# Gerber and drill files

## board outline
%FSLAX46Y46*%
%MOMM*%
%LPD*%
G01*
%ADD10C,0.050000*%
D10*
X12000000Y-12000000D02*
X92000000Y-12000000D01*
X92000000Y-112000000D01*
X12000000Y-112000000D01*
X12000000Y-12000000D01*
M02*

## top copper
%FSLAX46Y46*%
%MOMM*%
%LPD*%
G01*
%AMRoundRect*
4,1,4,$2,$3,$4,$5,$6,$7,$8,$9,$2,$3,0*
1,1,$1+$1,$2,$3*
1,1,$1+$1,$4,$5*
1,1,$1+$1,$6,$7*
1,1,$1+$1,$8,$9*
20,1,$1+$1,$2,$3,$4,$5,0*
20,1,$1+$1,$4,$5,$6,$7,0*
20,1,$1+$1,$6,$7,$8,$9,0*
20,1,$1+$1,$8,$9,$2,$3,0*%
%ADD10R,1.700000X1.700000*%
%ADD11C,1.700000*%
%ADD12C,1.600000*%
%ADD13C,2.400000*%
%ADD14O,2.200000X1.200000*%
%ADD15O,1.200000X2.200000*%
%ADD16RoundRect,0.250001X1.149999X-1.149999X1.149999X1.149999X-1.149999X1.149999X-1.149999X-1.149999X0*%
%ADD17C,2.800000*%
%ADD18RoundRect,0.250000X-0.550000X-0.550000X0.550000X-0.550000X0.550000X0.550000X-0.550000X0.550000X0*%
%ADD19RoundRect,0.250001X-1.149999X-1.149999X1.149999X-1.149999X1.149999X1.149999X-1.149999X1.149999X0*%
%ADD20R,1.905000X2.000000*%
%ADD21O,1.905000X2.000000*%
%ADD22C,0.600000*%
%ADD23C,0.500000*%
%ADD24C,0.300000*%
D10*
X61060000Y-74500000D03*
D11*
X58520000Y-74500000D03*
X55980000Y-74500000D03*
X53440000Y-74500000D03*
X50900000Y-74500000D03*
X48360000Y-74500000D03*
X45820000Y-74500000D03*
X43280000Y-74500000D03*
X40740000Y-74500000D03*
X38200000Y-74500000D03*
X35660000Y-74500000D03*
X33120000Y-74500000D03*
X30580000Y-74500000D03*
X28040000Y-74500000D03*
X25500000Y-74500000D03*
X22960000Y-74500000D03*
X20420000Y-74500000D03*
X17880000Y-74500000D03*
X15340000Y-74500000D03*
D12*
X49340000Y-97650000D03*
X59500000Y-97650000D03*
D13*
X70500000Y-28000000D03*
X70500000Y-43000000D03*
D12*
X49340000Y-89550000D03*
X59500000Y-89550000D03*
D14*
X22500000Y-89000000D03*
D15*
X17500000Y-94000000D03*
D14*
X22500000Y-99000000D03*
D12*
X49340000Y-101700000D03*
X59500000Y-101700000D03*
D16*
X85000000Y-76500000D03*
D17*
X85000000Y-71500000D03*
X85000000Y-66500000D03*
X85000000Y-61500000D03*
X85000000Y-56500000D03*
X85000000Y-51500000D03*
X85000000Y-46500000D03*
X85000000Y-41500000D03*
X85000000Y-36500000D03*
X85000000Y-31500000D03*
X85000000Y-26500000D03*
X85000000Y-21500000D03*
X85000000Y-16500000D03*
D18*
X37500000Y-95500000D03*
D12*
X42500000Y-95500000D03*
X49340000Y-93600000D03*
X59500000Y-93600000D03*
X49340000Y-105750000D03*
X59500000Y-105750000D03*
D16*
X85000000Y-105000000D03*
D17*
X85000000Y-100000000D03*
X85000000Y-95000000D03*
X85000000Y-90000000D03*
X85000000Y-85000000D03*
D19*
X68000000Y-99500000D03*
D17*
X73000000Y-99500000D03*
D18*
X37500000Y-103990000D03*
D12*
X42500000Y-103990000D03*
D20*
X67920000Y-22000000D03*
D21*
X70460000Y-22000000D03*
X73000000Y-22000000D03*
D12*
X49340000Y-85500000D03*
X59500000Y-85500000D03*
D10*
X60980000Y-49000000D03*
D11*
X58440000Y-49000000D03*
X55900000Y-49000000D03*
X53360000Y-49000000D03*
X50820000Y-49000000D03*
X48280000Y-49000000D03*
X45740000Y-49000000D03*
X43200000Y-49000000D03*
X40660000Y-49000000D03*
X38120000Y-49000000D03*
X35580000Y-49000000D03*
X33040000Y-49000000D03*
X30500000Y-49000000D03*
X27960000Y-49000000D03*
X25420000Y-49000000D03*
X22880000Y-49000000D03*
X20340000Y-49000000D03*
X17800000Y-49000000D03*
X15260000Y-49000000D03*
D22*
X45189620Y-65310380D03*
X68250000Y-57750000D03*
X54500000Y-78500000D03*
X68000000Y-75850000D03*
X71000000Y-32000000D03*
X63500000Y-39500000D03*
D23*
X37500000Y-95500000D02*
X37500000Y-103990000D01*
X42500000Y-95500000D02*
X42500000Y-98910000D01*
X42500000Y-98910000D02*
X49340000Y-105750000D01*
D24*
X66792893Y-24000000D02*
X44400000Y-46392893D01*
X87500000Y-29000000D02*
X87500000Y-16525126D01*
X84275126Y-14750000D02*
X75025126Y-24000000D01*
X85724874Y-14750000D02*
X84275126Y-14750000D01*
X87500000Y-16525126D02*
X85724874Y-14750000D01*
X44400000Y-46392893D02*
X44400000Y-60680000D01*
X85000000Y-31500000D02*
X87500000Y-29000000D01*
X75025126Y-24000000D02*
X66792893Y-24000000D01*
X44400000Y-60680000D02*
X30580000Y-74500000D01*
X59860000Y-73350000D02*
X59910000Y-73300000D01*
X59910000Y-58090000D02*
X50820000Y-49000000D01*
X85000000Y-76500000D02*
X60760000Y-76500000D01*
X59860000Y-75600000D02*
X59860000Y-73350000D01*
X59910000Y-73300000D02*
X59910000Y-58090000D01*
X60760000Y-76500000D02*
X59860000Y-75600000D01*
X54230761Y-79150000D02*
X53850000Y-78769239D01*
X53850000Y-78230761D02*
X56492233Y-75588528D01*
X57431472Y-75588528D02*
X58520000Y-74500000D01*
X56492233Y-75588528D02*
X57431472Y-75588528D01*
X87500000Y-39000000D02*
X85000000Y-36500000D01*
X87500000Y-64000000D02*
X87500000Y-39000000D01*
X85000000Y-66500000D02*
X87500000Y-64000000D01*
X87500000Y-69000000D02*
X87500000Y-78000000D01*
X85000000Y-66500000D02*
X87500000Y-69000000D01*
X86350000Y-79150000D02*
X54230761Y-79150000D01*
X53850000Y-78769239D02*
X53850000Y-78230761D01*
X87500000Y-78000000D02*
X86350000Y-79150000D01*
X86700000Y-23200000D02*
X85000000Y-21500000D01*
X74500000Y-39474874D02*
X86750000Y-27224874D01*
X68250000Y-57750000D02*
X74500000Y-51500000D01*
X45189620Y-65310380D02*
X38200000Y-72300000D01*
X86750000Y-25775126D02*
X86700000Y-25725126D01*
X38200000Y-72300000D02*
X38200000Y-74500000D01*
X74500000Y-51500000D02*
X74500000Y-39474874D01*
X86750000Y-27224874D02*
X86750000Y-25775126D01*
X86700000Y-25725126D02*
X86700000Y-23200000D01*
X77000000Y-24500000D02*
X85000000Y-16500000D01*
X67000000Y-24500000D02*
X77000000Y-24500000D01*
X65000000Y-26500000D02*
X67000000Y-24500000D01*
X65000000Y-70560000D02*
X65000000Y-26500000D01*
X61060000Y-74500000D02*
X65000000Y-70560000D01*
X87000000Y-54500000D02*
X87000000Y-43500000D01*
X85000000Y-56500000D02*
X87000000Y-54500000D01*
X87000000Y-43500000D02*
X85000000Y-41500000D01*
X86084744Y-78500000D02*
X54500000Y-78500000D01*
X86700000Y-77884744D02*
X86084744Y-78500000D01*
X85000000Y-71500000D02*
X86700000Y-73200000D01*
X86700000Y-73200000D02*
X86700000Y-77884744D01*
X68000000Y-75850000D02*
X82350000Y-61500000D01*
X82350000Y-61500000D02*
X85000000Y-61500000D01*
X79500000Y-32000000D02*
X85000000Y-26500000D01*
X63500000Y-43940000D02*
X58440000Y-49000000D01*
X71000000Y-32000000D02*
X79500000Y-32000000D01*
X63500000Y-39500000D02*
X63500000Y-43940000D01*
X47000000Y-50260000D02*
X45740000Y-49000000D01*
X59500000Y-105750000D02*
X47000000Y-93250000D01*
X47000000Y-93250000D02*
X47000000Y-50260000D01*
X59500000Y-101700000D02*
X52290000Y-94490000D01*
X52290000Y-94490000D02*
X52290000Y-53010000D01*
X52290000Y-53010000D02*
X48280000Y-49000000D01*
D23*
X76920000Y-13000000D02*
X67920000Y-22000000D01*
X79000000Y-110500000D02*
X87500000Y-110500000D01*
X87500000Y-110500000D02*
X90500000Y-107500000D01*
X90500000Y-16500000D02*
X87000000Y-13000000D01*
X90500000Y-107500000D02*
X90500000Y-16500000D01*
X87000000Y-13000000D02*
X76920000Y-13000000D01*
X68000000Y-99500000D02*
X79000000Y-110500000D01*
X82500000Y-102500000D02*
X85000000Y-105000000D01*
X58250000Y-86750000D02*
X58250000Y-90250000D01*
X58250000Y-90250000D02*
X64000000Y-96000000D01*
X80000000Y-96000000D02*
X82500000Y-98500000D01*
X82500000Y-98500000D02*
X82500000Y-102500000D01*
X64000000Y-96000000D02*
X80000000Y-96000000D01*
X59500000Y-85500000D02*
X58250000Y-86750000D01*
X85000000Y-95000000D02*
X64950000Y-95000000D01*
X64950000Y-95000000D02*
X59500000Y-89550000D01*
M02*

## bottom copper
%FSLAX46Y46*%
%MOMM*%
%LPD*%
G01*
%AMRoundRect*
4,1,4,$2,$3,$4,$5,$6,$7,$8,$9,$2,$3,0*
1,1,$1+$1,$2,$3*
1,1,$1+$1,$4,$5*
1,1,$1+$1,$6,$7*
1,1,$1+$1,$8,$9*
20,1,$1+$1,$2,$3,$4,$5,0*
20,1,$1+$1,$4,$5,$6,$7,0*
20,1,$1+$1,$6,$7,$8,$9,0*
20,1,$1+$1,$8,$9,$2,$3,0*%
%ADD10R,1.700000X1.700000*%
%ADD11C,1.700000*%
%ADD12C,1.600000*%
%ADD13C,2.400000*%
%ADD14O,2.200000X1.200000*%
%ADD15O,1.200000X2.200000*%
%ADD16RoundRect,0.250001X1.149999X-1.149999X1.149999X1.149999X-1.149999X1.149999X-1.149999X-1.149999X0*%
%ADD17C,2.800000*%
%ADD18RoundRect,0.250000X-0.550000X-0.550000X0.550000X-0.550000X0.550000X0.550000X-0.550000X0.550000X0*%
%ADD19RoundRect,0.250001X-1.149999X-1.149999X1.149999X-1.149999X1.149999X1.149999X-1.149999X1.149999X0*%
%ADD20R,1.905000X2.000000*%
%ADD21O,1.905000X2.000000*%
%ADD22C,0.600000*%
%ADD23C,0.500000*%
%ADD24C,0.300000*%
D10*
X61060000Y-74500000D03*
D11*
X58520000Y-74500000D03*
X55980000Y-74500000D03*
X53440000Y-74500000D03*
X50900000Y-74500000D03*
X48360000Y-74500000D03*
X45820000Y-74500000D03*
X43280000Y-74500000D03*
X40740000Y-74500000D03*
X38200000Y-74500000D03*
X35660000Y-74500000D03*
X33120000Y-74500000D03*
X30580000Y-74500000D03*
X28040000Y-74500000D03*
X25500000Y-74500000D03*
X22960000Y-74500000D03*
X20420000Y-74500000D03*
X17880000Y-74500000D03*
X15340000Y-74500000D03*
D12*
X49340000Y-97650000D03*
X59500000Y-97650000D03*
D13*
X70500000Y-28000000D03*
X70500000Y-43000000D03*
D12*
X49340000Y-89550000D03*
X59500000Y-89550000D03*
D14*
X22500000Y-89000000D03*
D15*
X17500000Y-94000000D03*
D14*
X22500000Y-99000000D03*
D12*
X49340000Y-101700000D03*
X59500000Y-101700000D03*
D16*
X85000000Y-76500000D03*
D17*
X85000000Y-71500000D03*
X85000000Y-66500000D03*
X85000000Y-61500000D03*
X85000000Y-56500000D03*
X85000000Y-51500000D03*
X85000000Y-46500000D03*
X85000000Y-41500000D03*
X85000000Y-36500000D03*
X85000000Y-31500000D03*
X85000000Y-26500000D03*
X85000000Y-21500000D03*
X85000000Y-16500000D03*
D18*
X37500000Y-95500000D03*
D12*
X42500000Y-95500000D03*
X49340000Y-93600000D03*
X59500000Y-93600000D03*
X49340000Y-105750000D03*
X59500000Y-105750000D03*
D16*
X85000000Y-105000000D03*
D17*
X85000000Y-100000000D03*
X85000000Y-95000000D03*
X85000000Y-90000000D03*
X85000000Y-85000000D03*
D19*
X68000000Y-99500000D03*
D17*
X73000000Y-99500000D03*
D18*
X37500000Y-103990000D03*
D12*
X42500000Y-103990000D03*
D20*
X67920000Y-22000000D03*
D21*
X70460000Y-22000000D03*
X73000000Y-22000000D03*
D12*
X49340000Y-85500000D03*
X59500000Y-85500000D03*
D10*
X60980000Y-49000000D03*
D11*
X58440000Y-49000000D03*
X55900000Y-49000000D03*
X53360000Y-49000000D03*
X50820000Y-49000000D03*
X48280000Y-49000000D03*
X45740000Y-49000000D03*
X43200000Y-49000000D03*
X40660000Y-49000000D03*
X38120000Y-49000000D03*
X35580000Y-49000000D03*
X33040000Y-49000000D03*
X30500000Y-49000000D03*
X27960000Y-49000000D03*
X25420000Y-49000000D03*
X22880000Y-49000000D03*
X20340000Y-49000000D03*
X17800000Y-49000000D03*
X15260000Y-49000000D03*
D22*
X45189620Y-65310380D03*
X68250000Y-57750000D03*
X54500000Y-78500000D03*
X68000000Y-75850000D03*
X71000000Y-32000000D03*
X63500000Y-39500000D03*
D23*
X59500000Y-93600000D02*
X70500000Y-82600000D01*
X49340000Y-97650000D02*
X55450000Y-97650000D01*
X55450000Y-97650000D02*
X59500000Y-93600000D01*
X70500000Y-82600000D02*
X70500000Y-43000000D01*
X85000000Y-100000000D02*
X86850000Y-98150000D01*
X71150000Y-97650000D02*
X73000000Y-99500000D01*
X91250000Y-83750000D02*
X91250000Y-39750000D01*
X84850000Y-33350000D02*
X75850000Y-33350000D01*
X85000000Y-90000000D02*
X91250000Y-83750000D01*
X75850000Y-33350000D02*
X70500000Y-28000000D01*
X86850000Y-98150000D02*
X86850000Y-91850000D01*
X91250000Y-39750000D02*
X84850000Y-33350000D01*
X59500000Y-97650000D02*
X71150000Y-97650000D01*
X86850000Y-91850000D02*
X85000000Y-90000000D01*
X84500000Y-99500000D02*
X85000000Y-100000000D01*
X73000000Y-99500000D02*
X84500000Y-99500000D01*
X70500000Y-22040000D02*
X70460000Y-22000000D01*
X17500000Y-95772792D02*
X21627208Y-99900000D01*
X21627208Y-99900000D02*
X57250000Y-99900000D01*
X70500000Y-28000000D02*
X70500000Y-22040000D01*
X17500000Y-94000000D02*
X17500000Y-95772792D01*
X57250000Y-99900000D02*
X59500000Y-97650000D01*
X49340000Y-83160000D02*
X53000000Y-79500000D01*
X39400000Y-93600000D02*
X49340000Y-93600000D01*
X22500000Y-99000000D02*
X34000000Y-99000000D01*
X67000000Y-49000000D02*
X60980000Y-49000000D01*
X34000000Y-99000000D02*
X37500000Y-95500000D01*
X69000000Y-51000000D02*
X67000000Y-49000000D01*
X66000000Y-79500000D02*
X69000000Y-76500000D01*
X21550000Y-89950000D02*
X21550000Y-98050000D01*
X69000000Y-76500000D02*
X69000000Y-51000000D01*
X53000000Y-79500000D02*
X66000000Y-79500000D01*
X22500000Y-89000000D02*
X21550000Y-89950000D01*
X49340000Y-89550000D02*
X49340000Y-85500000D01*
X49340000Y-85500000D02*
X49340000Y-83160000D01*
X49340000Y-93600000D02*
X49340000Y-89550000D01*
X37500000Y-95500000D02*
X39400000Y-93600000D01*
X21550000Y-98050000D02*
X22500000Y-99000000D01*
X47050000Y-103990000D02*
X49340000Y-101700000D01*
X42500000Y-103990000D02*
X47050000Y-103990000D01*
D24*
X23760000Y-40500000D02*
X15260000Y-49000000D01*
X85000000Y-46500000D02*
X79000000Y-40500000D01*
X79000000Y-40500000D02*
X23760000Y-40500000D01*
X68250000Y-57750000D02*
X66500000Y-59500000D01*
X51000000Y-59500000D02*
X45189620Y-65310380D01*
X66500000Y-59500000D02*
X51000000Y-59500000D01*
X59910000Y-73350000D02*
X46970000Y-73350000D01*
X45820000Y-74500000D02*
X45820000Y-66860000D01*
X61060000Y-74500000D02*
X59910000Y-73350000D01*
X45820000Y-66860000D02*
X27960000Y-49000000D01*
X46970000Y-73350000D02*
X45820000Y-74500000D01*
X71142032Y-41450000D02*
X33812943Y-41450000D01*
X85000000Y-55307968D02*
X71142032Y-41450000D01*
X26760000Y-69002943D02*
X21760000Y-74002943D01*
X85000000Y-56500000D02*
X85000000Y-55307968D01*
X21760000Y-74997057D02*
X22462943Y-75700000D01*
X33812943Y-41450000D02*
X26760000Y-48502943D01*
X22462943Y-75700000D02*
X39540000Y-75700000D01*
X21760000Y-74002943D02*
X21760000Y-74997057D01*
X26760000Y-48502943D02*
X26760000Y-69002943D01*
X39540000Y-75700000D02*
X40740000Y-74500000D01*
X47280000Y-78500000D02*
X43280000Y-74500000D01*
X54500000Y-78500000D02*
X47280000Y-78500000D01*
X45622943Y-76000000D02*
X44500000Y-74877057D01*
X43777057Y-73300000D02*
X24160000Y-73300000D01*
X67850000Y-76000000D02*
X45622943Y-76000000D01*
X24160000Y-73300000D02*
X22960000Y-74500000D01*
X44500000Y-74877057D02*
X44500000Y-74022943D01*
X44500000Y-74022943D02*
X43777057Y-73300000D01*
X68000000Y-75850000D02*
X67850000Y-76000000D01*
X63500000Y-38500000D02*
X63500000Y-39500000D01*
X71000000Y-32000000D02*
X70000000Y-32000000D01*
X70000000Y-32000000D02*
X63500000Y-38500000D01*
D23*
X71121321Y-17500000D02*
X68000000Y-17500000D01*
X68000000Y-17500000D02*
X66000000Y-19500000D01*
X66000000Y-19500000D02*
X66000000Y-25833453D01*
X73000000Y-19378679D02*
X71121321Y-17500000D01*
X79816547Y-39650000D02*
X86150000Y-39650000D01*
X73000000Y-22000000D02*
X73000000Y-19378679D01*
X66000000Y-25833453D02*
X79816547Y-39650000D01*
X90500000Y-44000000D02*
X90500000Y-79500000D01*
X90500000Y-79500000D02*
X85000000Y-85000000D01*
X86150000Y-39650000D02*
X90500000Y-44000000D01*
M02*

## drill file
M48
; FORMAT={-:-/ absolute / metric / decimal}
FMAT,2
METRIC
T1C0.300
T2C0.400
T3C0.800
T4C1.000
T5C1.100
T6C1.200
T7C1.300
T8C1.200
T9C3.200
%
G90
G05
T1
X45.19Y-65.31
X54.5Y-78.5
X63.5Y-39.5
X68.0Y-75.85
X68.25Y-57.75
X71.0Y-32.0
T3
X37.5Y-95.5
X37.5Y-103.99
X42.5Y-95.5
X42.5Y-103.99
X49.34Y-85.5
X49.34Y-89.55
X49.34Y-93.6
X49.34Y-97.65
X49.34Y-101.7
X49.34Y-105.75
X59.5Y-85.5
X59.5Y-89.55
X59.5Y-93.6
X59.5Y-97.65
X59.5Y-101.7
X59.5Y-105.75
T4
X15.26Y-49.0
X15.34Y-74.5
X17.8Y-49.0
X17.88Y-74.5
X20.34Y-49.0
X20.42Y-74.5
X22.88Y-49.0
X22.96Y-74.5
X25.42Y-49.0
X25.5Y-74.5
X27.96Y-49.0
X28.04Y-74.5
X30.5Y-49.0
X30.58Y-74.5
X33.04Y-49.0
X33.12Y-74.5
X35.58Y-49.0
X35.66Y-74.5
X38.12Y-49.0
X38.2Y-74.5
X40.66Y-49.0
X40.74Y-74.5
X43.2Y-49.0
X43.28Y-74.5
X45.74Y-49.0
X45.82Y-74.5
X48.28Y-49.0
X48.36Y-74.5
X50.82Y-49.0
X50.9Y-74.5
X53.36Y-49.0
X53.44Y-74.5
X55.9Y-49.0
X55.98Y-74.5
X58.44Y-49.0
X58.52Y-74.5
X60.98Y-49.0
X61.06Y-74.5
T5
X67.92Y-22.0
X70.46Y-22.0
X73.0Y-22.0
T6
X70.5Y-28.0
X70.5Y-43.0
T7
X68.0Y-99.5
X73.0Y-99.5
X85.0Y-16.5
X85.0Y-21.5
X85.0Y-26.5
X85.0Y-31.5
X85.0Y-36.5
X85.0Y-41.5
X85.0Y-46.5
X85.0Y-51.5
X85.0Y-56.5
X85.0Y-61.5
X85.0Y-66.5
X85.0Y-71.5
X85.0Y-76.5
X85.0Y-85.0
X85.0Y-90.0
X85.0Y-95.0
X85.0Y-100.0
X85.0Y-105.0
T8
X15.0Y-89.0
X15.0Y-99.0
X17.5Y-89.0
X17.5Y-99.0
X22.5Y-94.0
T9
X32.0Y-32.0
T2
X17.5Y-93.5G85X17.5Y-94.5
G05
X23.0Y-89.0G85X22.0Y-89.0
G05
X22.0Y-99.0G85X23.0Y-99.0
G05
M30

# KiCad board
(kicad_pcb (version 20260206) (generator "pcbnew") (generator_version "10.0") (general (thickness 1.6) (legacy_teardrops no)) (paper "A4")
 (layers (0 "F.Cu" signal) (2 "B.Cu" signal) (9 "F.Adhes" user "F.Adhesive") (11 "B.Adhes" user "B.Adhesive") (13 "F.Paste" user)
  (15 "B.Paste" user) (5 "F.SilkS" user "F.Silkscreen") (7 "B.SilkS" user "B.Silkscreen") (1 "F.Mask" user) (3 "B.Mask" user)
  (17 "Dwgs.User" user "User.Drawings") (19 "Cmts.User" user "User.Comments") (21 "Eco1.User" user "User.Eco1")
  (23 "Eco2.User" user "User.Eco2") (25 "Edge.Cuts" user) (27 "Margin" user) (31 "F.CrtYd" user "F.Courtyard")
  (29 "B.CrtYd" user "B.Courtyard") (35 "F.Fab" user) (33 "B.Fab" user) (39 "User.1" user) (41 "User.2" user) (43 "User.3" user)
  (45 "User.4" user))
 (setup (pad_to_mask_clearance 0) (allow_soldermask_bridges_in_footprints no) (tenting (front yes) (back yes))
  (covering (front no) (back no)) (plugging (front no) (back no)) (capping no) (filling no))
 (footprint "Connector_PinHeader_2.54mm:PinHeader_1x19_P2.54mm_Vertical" (layer "F.Cu") (at 61.06 74.5 -90)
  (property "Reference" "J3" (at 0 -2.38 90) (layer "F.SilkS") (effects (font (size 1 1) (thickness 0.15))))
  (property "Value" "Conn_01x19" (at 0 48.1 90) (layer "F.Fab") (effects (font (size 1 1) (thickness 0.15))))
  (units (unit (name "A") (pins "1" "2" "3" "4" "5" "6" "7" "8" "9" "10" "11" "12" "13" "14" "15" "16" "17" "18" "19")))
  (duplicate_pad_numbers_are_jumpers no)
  (pad "1" thru_hole rect (at 0 0 270) (size 1.7 1.7) (drill 1) (layers "*.Cu" "*.Mask") (remove_unused_layers no) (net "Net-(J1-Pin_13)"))
  (pad "2" thru_hole circle (at 0 2.54 270) (size 1.7 1.7) (drill 1) (layers "*.Cu" "*.Mask") (remove_unused_layers no)
   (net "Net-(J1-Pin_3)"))
  (pad "3" thru_hole circle (at 0 5.08 270) (size 1.7 1.7) (drill 1) (layers "*.Cu" "*.Mask") (remove_unused_layers no)
   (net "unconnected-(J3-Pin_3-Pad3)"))
  (pad "4" thru_hole circle (at 0 7.62 270) (size 1.7 1.7) (drill 1) (layers "*.Cu" "*.Mask") (remove_unused_layers no)
   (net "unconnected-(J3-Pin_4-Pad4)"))
  (pad "5" thru_hole circle (at 0 10.16 270) (size 1.7 1.7) (drill 1) (layers "*.Cu" "*.Mask") (remove_unused_layers no)
   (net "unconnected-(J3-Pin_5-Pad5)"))
  (pad "6" thru_hole circle (at 0 12.7 270) (size 1.7 1.7) (drill 1) (layers "*.Cu" "*.Mask") (remove_unused_layers no)
   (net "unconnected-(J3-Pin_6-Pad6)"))
  (pad "7" thru_hole circle (at 0 15.24 270) (size 1.7 1.7) (drill 1) (layers "*.Cu" "*.Mask") (remove_unused_layers no)
   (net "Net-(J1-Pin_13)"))
  (pad "8" thru_hole circle (at 0 17.78 270) (size 1.7 1.7) (drill 1) (layers "*.Cu" "*.Mask") (remove_unused_layers no)
   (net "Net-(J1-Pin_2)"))
  (pad "9" thru_hole circle (at 0 20.32 270) (size 1.7 1.7) (drill 1) (layers "*.Cu" "*.Mask") (remove_unused_layers no)
   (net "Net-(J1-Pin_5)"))
  (pad "10" thru_hole circle (at 0 22.86 270) (size 1.7 1.7) (drill 1) (layers "*.Cu" "*.Mask") (remove_unused_layers no)
   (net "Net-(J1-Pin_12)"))
  (pad "11" thru_hole circle (at 0 25.4 270) (size 1.7 1.7) (drill 1) (layers "*.Cu" "*.Mask") (remove_unused_layers no)
   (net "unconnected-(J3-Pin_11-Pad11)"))
  (pad "12" thru_hole circle (at 0 27.94 270) (size 1.7 1.7) (drill 1) (layers "*.Cu" "*.Mask") (remove_unused_layers no)
   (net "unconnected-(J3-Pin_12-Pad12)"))
  (pad "13" thru_hole circle (at 0 30.48 270) (size 1.7 1.7) (drill 1) (layers "*.Cu" "*.Mask") (remove_unused_layers no)
   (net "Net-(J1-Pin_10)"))
  (pad "14" thru_hole circle (at 0 33.02 270) (size 1.7 1.7) (drill 1) (layers "*.Cu" "*.Mask") (remove_unused_layers no)
   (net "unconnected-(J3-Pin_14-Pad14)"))
  (pad "15" thru_hole circle (at 0 35.56 270) (size 1.7 1.7) (drill 1) (layers "*.Cu" "*.Mask") (remove_unused_layers no)
   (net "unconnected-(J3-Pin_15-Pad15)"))
  (pad "16" thru_hole circle (at 0 38.1 270) (size 1.7 1.7) (drill 1) (layers "*.Cu" "*.Mask") (remove_unused_layers no)
   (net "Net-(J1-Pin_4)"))
  (pad "17" thru_hole circle (at 0 40.64 270) (size 1.7 1.7) (drill 1) (layers "*.Cu" "*.Mask") (remove_unused_layers no)
   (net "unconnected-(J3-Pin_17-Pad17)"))
  (pad "18" thru_hole circle (at 0 43.18 270) (size 1.7 1.7) (drill 1) (layers "*.Cu" "*.Mask") (remove_unused_layers no)
   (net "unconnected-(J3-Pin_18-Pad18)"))
  (pad "19" thru_hole circle (at 0 45.72 270) (size 1.7 1.7) (drill 1) (layers "*.Cu" "*.Mask") (remove_unused_layers no)
   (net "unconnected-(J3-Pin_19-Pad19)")))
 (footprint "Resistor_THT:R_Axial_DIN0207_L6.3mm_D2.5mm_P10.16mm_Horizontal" (layer "F.Cu") (at 49.34 97.65)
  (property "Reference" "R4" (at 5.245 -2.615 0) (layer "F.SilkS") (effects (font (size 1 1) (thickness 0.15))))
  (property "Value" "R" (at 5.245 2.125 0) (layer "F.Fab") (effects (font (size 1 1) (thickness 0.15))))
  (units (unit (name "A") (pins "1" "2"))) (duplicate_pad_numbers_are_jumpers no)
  (pad "1" thru_hole circle (at 0 0) (size 1.6 1.6) (drill 0.8) (layers "*.Cu" "*.Mask") (remove_unused_layers no) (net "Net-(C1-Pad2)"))
  (pad "2" thru_hole circle (at 10.16 0) (size 1.6 1.6) (drill 0.8) (layers "*.Cu" "*.Mask") (remove_unused_layers no) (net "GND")))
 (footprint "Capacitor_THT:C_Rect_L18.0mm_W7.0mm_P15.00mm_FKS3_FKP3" (layer "F.Cu") (at 70.5 28 -90)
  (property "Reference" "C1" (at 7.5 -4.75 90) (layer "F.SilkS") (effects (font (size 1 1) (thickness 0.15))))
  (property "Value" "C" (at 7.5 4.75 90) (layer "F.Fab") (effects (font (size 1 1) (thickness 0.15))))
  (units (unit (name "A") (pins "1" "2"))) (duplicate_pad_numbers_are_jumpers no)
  (pad "1" thru_hole circle (at 0 0 270) (size 2.4 2.4) (drill 1.2) (layers "*.Cu" "*.Mask") (remove_unused_layers no) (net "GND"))
  (pad "2" thru_hole circle (at 15 0 270) (size 2.4 2.4) (drill 1.2) (layers "*.Cu" "*.Mask") (remove_unused_layers no)
   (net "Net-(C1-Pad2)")))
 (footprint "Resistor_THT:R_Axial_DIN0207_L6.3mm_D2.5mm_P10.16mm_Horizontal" (layer "F.Cu") (at 49.34 89.55)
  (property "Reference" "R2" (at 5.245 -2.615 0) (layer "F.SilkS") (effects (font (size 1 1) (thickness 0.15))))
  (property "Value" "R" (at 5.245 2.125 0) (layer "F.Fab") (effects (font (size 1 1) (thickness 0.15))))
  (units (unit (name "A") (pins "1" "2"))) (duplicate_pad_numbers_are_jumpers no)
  (pad "1" thru_hole circle (at 0 0) (size 1.6 1.6) (drill 0.8) (layers "*.Cu" "*.Mask") (remove_unused_layers no) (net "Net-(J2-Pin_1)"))
  (pad "2" thru_hole circle (at 10.16 0) (size 1.6 1.6) (drill 0.8) (layers "*.Cu" "*.Mask") (remove_unused_layers no) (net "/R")))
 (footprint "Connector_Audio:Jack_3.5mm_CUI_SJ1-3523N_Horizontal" (layer "F.Cu") (at 17.5 94 -90)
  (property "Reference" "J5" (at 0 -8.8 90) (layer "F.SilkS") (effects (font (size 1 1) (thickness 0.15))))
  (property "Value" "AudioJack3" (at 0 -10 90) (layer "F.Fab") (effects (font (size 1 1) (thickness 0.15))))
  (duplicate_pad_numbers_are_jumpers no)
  (pad "" np_thru_hole circle (at -5 0 270) (size 1.2 1.2) (drill 1.2) (layers "*.Cu" "*.Mask"))
  (pad "" np_thru_hole circle (at -5 2.5 270) (size 1.2 1.2) (drill 1.2) (layers "*.Cu" "*.Mask"))
  (pad "" np_thru_hole circle (at 0 -5 270) (size 1.2 1.2) (drill 1.2) (layers "*.Cu" "*.Mask"))
  (pad "" np_thru_hole circle (at 5 0 270) (size 1.2 1.2) (drill 1.2) (layers "*.Cu" "*.Mask"))
  (pad "" np_thru_hole circle (at 5 2.5 270) (size 1.2 1.2) (drill 1.2) (layers "*.Cu" "*.Mask"))
  (pad "R" thru_hole oval (at -5 -5 270) (size 1.2 2.2) (drill oval 0.4 1.4) (layers "*.Cu" "*.Mask") (remove_unused_layers no)
   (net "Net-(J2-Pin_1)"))
  (pad "S" thru_hole oval (at 0 0 270) (size 2.2 1.2) (drill oval 1.4 0.4) (layers "*.Cu" "*.Mask") (remove_unused_layers no) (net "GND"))
  (pad "T" thru_hole oval (at 5 -5 90) (size 1.2 2.2) (drill oval 0.4 1.4) (layers "*.Cu" "*.Mask") (remove_unused_layers no)
   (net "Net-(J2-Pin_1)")))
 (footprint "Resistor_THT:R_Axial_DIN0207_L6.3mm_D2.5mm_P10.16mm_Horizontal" (layer "F.Cu") (at 49.34 101.7)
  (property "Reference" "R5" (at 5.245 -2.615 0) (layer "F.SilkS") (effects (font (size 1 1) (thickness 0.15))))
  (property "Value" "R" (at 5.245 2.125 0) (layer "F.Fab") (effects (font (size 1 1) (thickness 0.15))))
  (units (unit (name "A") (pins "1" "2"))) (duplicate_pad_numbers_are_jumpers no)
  (pad "1" thru_hole circle (at 0 0) (size 1.6 1.6) (drill 0.8) (layers "*.Cu" "*.Mask") (remove_unused_layers no) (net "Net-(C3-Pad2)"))
  (pad "2" thru_hole circle (at 10.16 0) (size 1.6 1.6) (drill 0.8) (layers "*.Cu" "*.Mask") (remove_unused_layers no)
   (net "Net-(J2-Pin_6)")))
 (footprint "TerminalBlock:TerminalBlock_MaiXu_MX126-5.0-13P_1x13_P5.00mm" (layer "F.Cu") (at 85 76.5 90)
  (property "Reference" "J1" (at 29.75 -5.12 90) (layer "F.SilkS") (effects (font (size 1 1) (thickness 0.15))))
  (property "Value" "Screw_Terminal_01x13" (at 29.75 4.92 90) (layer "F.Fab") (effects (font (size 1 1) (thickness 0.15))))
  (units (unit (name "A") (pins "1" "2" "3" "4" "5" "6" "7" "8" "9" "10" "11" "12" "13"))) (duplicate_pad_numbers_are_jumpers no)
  (pad "1" thru_hole roundrect (at 0 0 90) (size 2.8 2.8) (drill 1.3) (layers "*.Cu" "*.Mask") (remove_unused_layers no)
   (roundrect_rratio 0.089286) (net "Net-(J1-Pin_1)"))
  (pad "2" thru_hole circle (at 5 0 90) (size 2.8 2.8) (drill 1.3) (layers "*.Cu" "*.Mask") (remove_unused_layers no) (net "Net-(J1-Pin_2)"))
  (pad "3" thru_hole circle (at 10 0 90) (size 2.8 2.8) (drill 1.3) (layers "*.Cu" "*.Mask") (remove_unused_layers no)
   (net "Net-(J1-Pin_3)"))
  (pad "4" thru_hole circle (at 15 0 90) (size 2.8 2.8) (drill 1.3) (layers "*.Cu" "*.Mask") (remove_unused_layers no)
   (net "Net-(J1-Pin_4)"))
  (pad "5" thru_hole circle (at 20 0 90) (size 2.8 2.8) (drill 1.3) (layers "*.Cu" "*.Mask") (remove_unused_layers no)
   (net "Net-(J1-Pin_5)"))
  (pad "6" thru_hole circle (at 25 0 90) (size 2.8 2.8) (drill 1.3) (layers "*.Cu" "*.Mask") (remove_unused_layers no)
   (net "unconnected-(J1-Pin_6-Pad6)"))
  (pad "7" thru_hole circle (at 30 0 90) (size 2.8 2.8) (drill 1.3) (layers "*.Cu" "*.Mask") (remove_unused_layers no)
   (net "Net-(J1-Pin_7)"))
  (pad "8" thru_hole circle (at 35 0 90) (size 2.8 2.8) (drill 1.3) (layers "*.Cu" "*.Mask") (remove_unused_layers no)
   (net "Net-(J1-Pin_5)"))
  (pad "9" thru_hole circle (at 40 0 90) (size 2.8 2.8) (drill 1.3) (layers "*.Cu" "*.Mask") (remove_unused_layers no)
   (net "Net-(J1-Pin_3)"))
  (pad "10" thru_hole circle (at 45 0 90) (size 2.8 2.8) (drill 1.3) (layers "*.Cu" "*.Mask") (remove_unused_layers no)
   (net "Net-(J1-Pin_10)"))
  (pad "11" thru_hole circle (at 50 0 90) (size 2.8 2.8) (drill 1.3) (layers "*.Cu" "*.Mask") (remove_unused_layers no)
   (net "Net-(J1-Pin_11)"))
  (pad "12" thru_hole circle (at 55 0 90) (size 2.8 2.8) (drill 1.3) (layers "*.Cu" "*.Mask") (remove_unused_layers no)
   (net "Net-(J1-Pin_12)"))
  (pad "13" thru_hole circle (at 60 0 90) (size 2.8 2.8) (drill 1.3) (layers "*.Cu" "*.Mask") (remove_unused_layers no)
   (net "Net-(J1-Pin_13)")))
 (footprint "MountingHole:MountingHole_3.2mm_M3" (layer "F.Cu") (at 32 32)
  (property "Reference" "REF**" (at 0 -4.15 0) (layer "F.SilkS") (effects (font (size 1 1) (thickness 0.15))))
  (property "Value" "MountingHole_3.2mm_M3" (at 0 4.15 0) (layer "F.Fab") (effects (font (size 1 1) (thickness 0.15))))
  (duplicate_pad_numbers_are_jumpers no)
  (pad "" np_thru_hole circle (at 0 0) (size 3.2 3.2) (drill 3.2) (layers "*.Cu" "*.Mask")))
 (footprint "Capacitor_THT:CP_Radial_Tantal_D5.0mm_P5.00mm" (layer "F.Cu") (at 37.5 95.5)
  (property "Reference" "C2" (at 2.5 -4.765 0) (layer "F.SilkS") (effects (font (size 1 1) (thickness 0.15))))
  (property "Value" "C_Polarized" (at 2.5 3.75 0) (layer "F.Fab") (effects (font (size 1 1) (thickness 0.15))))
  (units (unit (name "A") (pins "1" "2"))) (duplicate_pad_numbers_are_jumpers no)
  (pad "1" thru_hole roundrect (at 0 0) (size 1.6 1.6) (drill 0.8) (layers "*.Cu" "*.Mask") (remove_unused_layers no)
   (roundrect_rratio 0.15625) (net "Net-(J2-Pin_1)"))
  (pad "2" thru_hole circle (at 5 0) (size 1.6 1.6) (drill 0.8) (layers "*.Cu" "*.Mask") (remove_unused_layers no) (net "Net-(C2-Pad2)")))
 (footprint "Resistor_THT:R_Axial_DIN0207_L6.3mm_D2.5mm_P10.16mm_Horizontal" (layer "F.Cu") (at 49.34 93.6)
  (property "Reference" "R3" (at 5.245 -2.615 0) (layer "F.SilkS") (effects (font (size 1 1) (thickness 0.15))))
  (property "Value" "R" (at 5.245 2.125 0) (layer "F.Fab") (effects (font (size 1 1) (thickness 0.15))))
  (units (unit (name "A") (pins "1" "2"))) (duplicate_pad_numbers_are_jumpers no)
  (pad "1" thru_hole circle (at 0 0) (size 1.6 1.6) (drill 0.8) (layers "*.Cu" "*.Mask") (remove_unused_layers no) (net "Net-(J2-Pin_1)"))
  (pad "2" thru_hole circle (at 10.16 0) (size 1.6 1.6) (drill 0.8) (layers "*.Cu" "*.Mask") (remove_unused_layers no) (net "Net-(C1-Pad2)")))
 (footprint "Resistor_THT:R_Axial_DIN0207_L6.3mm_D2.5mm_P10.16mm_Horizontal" (layer "F.Cu") (at 49.34 105.75)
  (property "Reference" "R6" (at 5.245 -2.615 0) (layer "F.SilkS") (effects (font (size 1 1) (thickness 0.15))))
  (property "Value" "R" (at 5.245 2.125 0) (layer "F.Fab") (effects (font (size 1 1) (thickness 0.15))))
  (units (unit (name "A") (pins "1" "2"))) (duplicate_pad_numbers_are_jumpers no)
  (pad "1" thru_hole circle (at 0 0) (size 1.6 1.6) (drill 0.8) (layers "*.Cu" "*.Mask") (remove_unused_layers no) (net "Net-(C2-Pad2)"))
  (pad "2" thru_hole circle (at 10.16 0) (size 1.6 1.6) (drill 0.8) (layers "*.Cu" "*.Mask") (remove_unused_layers no)
   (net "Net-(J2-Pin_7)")))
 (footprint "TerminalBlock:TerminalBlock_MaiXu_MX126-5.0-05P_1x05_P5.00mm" (layer "F.Cu") (at 85 105 90)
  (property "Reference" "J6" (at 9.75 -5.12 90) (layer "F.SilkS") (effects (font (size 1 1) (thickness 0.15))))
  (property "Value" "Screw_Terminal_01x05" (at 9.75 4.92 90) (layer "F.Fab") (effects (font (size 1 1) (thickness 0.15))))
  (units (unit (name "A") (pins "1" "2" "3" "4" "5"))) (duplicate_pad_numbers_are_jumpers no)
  (pad "1" thru_hole roundrect (at 0 0 90) (size 2.8 2.8) (drill 1.3) (layers "*.Cu" "*.Mask") (remove_unused_layers no)
   (roundrect_rratio 0.089286) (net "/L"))
  (pad "2" thru_hole circle (at 5 0 90) (size 2.8 2.8) (drill 1.3) (layers "*.Cu" "*.Mask") (remove_unused_layers no) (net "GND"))
  (pad "3" thru_hole circle (at 10 0 90) (size 2.8 2.8) (drill 1.3) (layers "*.Cu" "*.Mask") (remove_unused_layers no) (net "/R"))
  (pad "4" thru_hole circle (at 15 0 90) (size 2.8 2.8) (drill 1.3) (layers "*.Cu" "*.Mask") (remove_unused_layers no) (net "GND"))
  (pad "5" thru_hole circle (at 20 0 90) (size 2.8 2.8) (drill 1.3) (layers "*.Cu" "*.Mask") (remove_unused_layers no) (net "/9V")))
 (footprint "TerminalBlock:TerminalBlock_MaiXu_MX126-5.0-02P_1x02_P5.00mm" (layer "F.Cu") (at 68 99.5)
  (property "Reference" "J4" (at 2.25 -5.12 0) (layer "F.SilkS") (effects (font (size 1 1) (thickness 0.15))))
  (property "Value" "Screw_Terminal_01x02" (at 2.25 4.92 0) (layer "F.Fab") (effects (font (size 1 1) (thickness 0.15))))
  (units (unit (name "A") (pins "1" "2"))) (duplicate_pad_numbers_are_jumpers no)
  (pad "1" thru_hole roundrect (at 0 0) (size 2.8 2.8) (drill 1.3) (layers "*.Cu" "*.Mask") (remove_unused_layers no)
   (roundrect_rratio 0.089286) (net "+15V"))
  (pad "2" thru_hole circle (at 5 0) (size 2.8 2.8) (drill 1.3) (layers "*.Cu" "*.Mask") (remove_unused_layers no) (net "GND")))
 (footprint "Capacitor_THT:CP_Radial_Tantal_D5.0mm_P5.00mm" (layer "F.Cu") (at 37.5 103.99)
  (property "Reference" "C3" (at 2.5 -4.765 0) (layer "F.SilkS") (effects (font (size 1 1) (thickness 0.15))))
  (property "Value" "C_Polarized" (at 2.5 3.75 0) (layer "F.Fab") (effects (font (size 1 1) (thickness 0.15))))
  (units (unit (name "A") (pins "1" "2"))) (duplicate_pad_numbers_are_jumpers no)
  (pad "1" thru_hole roundrect (at 0 0) (size 1.6 1.6) (drill 0.8) (layers "*.Cu" "*.Mask") (remove_unused_layers no)
   (roundrect_rratio 0.15625) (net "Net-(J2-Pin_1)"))
  (pad "2" thru_hole circle (at 5 0) (size 1.6 1.6) (drill 0.8) (layers "*.Cu" "*.Mask") (remove_unused_layers no) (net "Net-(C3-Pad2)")))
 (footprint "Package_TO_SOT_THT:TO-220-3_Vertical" (layer "F.Cu") (at 67.92 22)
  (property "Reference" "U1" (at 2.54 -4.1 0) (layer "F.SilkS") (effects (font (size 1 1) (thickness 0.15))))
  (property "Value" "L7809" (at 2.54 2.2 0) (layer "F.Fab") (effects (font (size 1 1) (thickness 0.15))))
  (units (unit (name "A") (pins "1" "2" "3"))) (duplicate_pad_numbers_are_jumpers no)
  (pad "1" thru_hole rect (at 0 0) (size 1.905 2) (drill 1.1) (layers "*.Cu" "*.Mask") (remove_unused_layers no) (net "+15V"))
  (pad "2" thru_hole oval (at 2.54 0) (size 1.905 2) (drill 1.1) (layers "*.Cu" "*.Mask") (remove_unused_layers no) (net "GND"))
  (pad "3" thru_hole oval (at 5.08 0) (size 1.905 2) (drill 1.1) (layers "*.Cu" "*.Mask") (remove_unused_layers no) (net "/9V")))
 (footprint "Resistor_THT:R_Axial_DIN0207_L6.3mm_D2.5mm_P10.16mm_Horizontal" (layer "F.Cu") (at 49.34 85.5)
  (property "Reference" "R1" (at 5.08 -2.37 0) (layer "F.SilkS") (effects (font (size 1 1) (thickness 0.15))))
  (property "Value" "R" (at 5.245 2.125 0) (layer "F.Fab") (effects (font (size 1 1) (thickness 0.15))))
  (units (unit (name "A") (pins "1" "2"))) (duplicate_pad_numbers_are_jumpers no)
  (pad "1" thru_hole circle (at 0 0) (size 1.6 1.6) (drill 0.8) (layers "*.Cu" "*.Mask") (remove_unused_layers no) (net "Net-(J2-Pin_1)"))
  (pad "2" thru_hole circle (at 10.16 0) (size 1.6 1.6) (drill 0.8) (layers "*.Cu" "*.Mask") (remove_unused_layers no) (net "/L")))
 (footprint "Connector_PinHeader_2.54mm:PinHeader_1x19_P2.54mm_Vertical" (layer "F.Cu") (at 60.98 49 -90)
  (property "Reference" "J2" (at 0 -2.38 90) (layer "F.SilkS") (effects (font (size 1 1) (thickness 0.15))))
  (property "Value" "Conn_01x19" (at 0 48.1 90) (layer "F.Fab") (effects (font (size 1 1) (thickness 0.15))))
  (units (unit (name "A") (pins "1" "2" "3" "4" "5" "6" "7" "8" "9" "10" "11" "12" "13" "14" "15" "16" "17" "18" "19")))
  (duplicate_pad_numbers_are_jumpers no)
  (pad "1" thru_hole rect (at 0 0 270) (size 1.7 1.7) (drill 1) (layers "*.Cu" "*.Mask") (remove_unused_layers no) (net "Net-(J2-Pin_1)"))
  (pad "2" thru_hole circle (at 0 2.54 270) (size 1.7 1.7) (drill 1) (layers "*.Cu" "*.Mask") (remove_unused_layers no)
   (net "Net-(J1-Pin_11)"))
  (pad "3" thru_hole circle (at 0 5.08 270) (size 1.7 1.7) (drill 1) (layers "*.Cu" "*.Mask") (remove_unused_layers no)
   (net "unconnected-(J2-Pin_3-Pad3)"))
  (pad "4" thru_hole circle (at 0 7.62 270) (size 1.7 1.7) (drill 1) (layers "*.Cu" "*.Mask") (remove_unused_layers no)
   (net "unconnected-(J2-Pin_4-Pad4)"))
  (pad "5" thru_hole circle (at 0 10.16 270) (size 1.7 1.7) (drill 1) (layers "*.Cu" "*.Mask") (remove_unused_layers no)
   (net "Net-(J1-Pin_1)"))
  (pad "6" thru_hole circle (at 0 12.7 270) (size 1.7 1.7) (drill 1) (layers "*.Cu" "*.Mask") (remove_unused_layers no)
   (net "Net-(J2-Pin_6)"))
  (pad "7" thru_hole circle (at 0 15.24 270) (size 1.7 1.7) (drill 1) (layers "*.Cu" "*.Mask") (remove_unused_layers no)
   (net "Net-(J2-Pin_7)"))
  (pad "8" thru_hole circle (at 0 17.78 270) (size 1.7 1.7) (drill 1) (layers "*.Cu" "*.Mask") (remove_unused_layers no)
   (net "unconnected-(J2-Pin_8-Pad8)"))
  (pad "9" thru_hole circle (at 0 20.32 270) (size 1.7 1.7) (drill 1) (layers "*.Cu" "*.Mask") (remove_unused_layers no)
   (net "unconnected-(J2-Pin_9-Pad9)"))
  (pad "10" thru_hole circle (at 0 22.86 270) (size 1.7 1.7) (drill 1) (layers "*.Cu" "*.Mask") (remove_unused_layers no)
   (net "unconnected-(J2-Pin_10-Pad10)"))
  (pad "11" thru_hole circle (at 0 25.4 270) (size 1.7 1.7) (drill 1) (layers "*.Cu" "*.Mask") (remove_unused_layers no)
   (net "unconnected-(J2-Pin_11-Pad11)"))
  (pad "12" thru_hole circle (at 0 27.94 270) (size 1.7 1.7) (drill 1) (layers "*.Cu" "*.Mask") (remove_unused_layers no)
   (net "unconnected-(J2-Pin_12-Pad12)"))
  (pad "13" thru_hole circle (at 0 30.48 270) (size 1.7 1.7) (drill 1) (layers "*.Cu" "*.Mask") (remove_unused_layers no)
   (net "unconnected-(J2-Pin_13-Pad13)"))
  (pad "14" thru_hole circle (at 0 33.02 270) (size 1.7 1.7) (drill 1) (layers "*.Cu" "*.Mask") (remove_unused_layers no)
   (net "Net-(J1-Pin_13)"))
  (pad "15" thru_hole circle (at 0 35.56 270) (size 1.7 1.7) (drill 1) (layers "*.Cu" "*.Mask") (remove_unused_layers no)
   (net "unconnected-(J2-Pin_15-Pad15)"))
  (pad "16" thru_hole circle (at 0 38.1 270) (size 1.7 1.7) (drill 1) (layers "*.Cu" "*.Mask") (remove_unused_layers no)
   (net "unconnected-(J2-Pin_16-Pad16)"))
  (pad "17" thru_hole circle (at 0 40.64 270) (size 1.7 1.7) (drill 1) (layers "*.Cu" "*.Mask") (remove_unused_layers no)
   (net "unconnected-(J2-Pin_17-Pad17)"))
  (pad "18" thru_hole circle (at 0 43.18 270) (size 1.7 1.7) (drill 1) (layers "*.Cu" "*.Mask") (remove_unused_layers no)
   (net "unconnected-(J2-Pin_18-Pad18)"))
  (pad "19" thru_hole circle (at 0 45.72 270) (size 1.7 1.7) (drill 1) (layers "*.Cu" "*.Mask") (remove_unused_layers no)
   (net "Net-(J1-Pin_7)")))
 (gr_rect (start 12 12) (end 92 112) (stroke (width 0.05) (type default)) (fill no) (layer "Edge.Cuts"))
 (segment (start 59.5 93.6) (end 70.5 82.6) (width 0.5) (layer "B.Cu") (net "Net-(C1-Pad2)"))
 (segment (start 49.34 97.65) (end 55.45 97.65) (width 0.5) (layer "B.Cu") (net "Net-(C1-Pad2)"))
 (segment (start 55.45 97.65) (end 59.5 93.6) (width 0.5) (layer "B.Cu") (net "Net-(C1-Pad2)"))
 (segment (start 70.5 82.6) (end 70.5 43) (width 0.5) (layer "B.Cu") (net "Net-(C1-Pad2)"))
 (segment (start 85 100) (end 86.85 98.15) (width 0.5) (layer "B.Cu") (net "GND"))
 (segment (start 71.15 97.65) (end 73 99.5) (width 0.5) (layer "B.Cu") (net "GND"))
 (segment (start 91.25 83.75) (end 91.25 39.75) (width 0.5) (layer "B.Cu") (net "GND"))
 (segment (start 84.85 33.35) (end 75.85 33.35) (width 0.5) (layer "B.Cu") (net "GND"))
 (segment (start 85 90) (end 91.25 83.75) (width 0.5) (layer "B.Cu") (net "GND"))
 (segment (start 75.85 33.35) (end 70.5 28) (width 0.5) (layer "B.Cu") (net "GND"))
 (segment (start 86.85 98.15) (end 86.85 91.85) (width 0.5) (layer "B.Cu") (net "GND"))
 (segment (start 91.25 39.75) (end 84.85 33.35) (width 0.5) (layer "B.Cu") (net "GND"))
 (segment (start 59.5 97.65) (end 71.15 97.65) (width 0.5) (layer "B.Cu") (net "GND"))
 (segment (start 86.85 91.85) (end 85 90) (width 0.5) (layer "B.Cu") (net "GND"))
 (segment (start 84.5 99.5) (end 85 100) (width 0.5) (layer "B.Cu") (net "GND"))
 (segment (start 73 99.5) (end 84.5 99.5) (width 0.5) (layer "B.Cu") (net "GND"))
 (segment (start 70.5 22.04) (end 70.46 22) (width 0.5) (layer "B.Cu") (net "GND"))
 (segment (start 17.5 95.772792) (end 21.627208 99.9) (width 0.5) (layer "B.Cu") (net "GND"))
 (segment (start 21.627208 99.9) (end 57.25 99.9) (width 0.5) (layer "B.Cu") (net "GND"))
 (segment (start 70.5 28) (end 70.5 22.04) (width 0.5) (layer "B.Cu") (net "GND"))
 (segment (start 17.5 94) (end 17.5 95.772792) (width 0.5) (layer "B.Cu") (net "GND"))
 (segment (start 57.25 99.9) (end 59.5 97.65) (width 0.5) (layer "B.Cu") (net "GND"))
 (segment (start 37.5 95.5) (end 37.5 103.99) (width 0.5) (layer "F.Cu") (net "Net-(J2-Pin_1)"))
 (segment (start 49.34 83.16) (end 53 79.5) (width 0.5) (layer "B.Cu") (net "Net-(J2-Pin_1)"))
 (segment (start 39.4 93.6) (end 49.34 93.6) (width 0.5) (layer "B.Cu") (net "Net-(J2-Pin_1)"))
 (segment (start 22.5 99) (end 34 99) (width 0.5) (layer "B.Cu") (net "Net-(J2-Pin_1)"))
 (segment (start 67 49) (end 60.98 49) (width 0.5) (layer "B.Cu") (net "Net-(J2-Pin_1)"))
 (segment (start 34 99) (end 37.5 95.5) (width 0.5) (layer "B.Cu") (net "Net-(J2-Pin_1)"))
 (segment (start 69 51) (end 67 49) (width 0.5) (layer "B.Cu") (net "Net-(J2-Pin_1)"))
 (segment (start 66 79.5) (end 69 76.5) (width 0.5) (layer "B.Cu") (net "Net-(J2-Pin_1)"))
 (segment (start 21.55 89.95) (end 21.55 98.05) (width 0.5) (layer "B.Cu") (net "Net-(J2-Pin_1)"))
 (segment (start 69 76.5) (end 69 51) (width 0.5) (layer "B.Cu") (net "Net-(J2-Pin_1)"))
 (segment (start 53 79.5) (end 66 79.5) (width 0.5) (layer "B.Cu") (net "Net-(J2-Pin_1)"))
 (segment (start 22.5 89) (end 21.55 89.95) (width 0.5) (layer "B.Cu") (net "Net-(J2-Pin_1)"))
 (segment (start 49.34 89.55) (end 49.34 85.5) (width 0.5) (layer "B.Cu") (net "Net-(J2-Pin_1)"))
 (segment (start 49.34 85.5) (end 49.34 83.16) (width 0.5) (layer "B.Cu") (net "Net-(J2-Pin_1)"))
 (segment (start 49.34 93.6) (end 49.34 89.55) (width 0.5) (layer "B.Cu") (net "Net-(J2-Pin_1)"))
 (segment (start 37.5 95.5) (end 39.4 93.6) (width 0.5) (layer "B.Cu") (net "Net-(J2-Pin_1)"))
 (segment (start 21.55 98.05) (end 22.5 99) (width 0.5) (layer "B.Cu") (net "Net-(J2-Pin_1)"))
 (segment (start 42.5 95.5) (end 42.5 98.91) (width 0.5) (layer "F.Cu") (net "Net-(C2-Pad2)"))
 (segment (start 42.5 98.91) (end 49.34 105.75) (width 0.5) (layer "F.Cu") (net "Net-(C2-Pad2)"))
 (segment (start 47.05 103.99) (end 49.34 101.7) (width 0.5) (layer "B.Cu") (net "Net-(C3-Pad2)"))
 (segment (start 42.5 103.99) (end 47.05 103.99) (width 0.5) (layer "B.Cu") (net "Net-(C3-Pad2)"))
 (segment (start 66.792893 24) (end 44.4 46.392893) (width 0.3) (layer "F.Cu") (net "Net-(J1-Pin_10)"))
 (segment (start 87.5 29) (end 87.5 16.525126) (width 0.3) (layer "F.Cu") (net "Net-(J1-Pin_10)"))
 (segment (start 84.275126 14.75) (end 75.025126 24) (width 0.3) (layer "F.Cu") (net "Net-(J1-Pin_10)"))
 (segment (start 85.724874 14.75) (end 84.275126 14.75) (width 0.3) (layer "F.Cu") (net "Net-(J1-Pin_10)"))
 (segment (start 87.5 16.525126) (end 85.724874 14.75) (width 0.3) (layer "F.Cu") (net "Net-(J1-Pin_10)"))
 (segment (start 44.4 46.392893) (end 44.4 60.68) (width 0.3) (layer "F.Cu") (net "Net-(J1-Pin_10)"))
 (segment (start 85 31.5) (end 87.5 29) (width 0.3) (layer "F.Cu") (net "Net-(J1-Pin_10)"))
 (segment (start 75.025126 24) (end 66.792893 24) (width 0.3) (layer "F.Cu") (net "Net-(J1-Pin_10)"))
 (segment (start 44.4 60.68) (end 30.58 74.5) (width 0.3) (layer "F.Cu") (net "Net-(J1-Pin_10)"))
 (segment (start 23.76 40.5) (end 15.26 49) (width 0.3) (layer "B.Cu") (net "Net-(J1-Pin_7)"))
 (segment (start 85 46.5) (end 79 40.5) (width 0.3) (layer "B.Cu") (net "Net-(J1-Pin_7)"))
 (segment (start 79 40.5) (end 23.76 40.5) (width 0.3) (layer "B.Cu") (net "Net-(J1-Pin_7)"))
 (segment (start 59.86 73.35) (end 59.91 73.3) (width 0.3) (layer "F.Cu") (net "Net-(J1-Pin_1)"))
 (segment (start 59.91 58.09) (end 50.82 49) (width 0.3) (layer "F.Cu") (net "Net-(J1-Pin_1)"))
 (segment (start 85 76.5) (end 60.76 76.5) (width 0.3) (layer "F.Cu") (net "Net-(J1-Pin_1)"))
 (segment (start 59.86 75.6) (end 59.86 73.35) (width 0.3) (layer "F.Cu") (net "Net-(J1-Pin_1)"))
 (segment (start 59.91 73.3) (end 59.91 58.09) (width 0.3) (layer "F.Cu") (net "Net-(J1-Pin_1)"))
 (segment (start 60.76 76.5) (end 59.86 75.6) (width 0.3) (layer "F.Cu") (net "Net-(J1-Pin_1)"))
 (segment (start 54.230761 79.15) (end 53.85 78.769239) (width 0.3) (layer "F.Cu") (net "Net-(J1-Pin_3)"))
 (segment (start 53.85 78.230761) (end 56.492233 75.588528) (width 0.3) (layer "F.Cu") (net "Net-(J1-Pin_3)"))
 (segment (start 57.431472 75.588528) (end 58.52 74.5) (width 0.3) (layer "F.Cu") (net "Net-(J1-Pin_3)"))
 (segment (start 56.492233 75.588528) (end 57.431472 75.588528) (width 0.3) (layer "F.Cu") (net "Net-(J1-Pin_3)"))
 (segment (start 87.5 39) (end 85 36.5) (width 0.3) (layer "F.Cu") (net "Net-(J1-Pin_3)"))
 (segment (start 87.5 64) (end 87.5 39) (width 0.3) (layer "F.Cu") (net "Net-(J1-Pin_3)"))
 (segment (start 85 66.5) (end 87.5 64) (width 0.3) (layer "F.Cu") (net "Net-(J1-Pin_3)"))
 (segment (start 87.5 69) (end 87.5 78) (width 0.3) (layer "F.Cu") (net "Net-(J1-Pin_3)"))
 (segment (start 85 66.5) (end 87.5 69) (width 0.3) (layer "F.Cu") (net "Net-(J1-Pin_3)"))
 (segment (start 86.35 79.15) (end 54.230761 79.15) (width 0.3) (layer "F.Cu") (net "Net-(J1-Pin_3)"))
 (segment (start 53.85 78.769239) (end 53.85 78.230761) (width 0.3) (layer "F.Cu") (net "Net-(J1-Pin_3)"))
 (segment (start 87.5 78) (end 86.35 79.15) (width 0.3) (layer "F.Cu") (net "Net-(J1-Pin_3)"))
 (segment (start 86.7 23.2) (end 85 21.5) (width 0.3) (layer "F.Cu") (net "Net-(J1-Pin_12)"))
 (segment (start 74.5 39.474874) (end 86.75 27.224874) (width 0.3) (layer "F.Cu") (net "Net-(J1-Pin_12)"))
 (segment (start 68.25 57.75) (end 74.5 51.5) (width 0.3) (layer "F.Cu") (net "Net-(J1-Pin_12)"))
 (segment (start 45.18962 65.31038) (end 38.2 72.3) (width 0.3) (layer "F.Cu") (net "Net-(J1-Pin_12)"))
 (segment (start 86.75 25.775126) (end 86.7 25.725126) (width 0.3) (layer "F.Cu") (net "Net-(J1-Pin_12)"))
 (segment (start 38.2 72.3) (end 38.2 74.5) (width 0.3) (layer "F.Cu") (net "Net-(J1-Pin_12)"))
 (segment (start 74.5 51.5) (end 74.5 39.474874) (width 0.3) (layer "F.Cu") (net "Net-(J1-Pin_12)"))
 (segment (start 86.75 27.224874) (end 86.75 25.775126) (width 0.3) (layer "F.Cu") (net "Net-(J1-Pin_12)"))
 (segment (start 86.7 25.725126) (end 86.7 23.2) (width 0.3) (layer "F.Cu") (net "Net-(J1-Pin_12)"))
 (via (at 45.18962 65.31038) (size 0.6) (drill 0.3) (layers "F.Cu" "B.Cu") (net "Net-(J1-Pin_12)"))
 (via (at 68.25 57.75) (size 0.6) (drill 0.3) (layers "F.Cu" "B.Cu") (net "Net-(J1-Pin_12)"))
 (segment (start 68.25 57.75) (end 66.5 59.5) (width 0.3) (layer "B.Cu") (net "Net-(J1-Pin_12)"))
 (segment (start 51 59.5) (end 45.18962 65.31038) (width 0.3) (layer "B.Cu") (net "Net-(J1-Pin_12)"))
 (segment (start 66.5 59.5) (end 51 59.5) (width 0.3) (layer "B.Cu") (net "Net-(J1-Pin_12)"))
 (segment (start 77 24.5) (end 85 16.5) (width 0.3) (layer "F.Cu") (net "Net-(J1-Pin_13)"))
 (segment (start 67 24.5) (end 77 24.5) (width 0.3) (layer "F.Cu") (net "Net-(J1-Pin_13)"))
 (segment (start 65 26.5) (end 67 24.5) (width 0.3) (layer "F.Cu") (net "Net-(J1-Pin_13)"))
 (segment (start 65 70.56) (end 65 26.5) (width 0.3) (layer "F.Cu") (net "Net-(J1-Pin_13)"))
 (segment (start 61.06 74.5) (end 65 70.56) (width 0.3) (layer "F.Cu") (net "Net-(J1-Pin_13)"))
 (segment (start 59.91 73.35) (end 46.97 73.35) (width 0.3) (layer "B.Cu") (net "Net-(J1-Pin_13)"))
 (segment (start 45.82 74.5) (end 45.82 66.86) (width 0.3) (layer "B.Cu") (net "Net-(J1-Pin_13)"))
 (segment (start 61.06 74.5) (end 59.91 73.35) (width 0.3) (layer "B.Cu") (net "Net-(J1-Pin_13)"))
 (segment (start 45.82 66.86) (end 27.96 49) (width 0.3) (layer "B.Cu") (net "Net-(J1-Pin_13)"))
 (segment (start 46.97 73.35) (end 45.82 74.5) (width 0.3) (layer "B.Cu") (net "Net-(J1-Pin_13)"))
 (segment (start 87 54.5) (end 87 43.5) (width 0.3) (layer "F.Cu") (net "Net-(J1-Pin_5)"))
 (segment (start 85 56.5) (end 87 54.5) (width 0.3) (layer "F.Cu") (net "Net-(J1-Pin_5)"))
 (segment (start 87 43.5) (end 85 41.5) (width 0.3) (layer "F.Cu") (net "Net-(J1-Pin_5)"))
 (segment (start 71.142032 41.45) (end 33.812943 41.45) (width 0.3) (layer "B.Cu") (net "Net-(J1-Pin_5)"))
 (segment (start 85 55.307968) (end 71.142032 41.45) (width 0.3) (layer "B.Cu") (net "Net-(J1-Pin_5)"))
 (segment (start 26.76 69.002943) (end 21.76 74.002943) (width 0.3) (layer "B.Cu") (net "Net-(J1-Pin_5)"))
 (segment (start 85 56.5) (end 85 55.307968) (width 0.3) (layer "B.Cu") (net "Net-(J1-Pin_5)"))
 (segment (start 21.76 74.997057) (end 22.462943 75.7) (width 0.3) (layer "B.Cu") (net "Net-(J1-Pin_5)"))
 (segment (start 33.812943 41.45) (end 26.76 48.502943) (width 0.3) (layer "B.Cu") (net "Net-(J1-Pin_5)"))
 (segment (start 22.462943 75.7) (end 39.54 75.7) (width 0.3) (layer "B.Cu") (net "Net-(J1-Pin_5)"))
 (segment (start 21.76 74.002943) (end 21.76 74.997057) (width 0.3) (layer "B.Cu") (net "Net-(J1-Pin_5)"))
 (segment (start 26.76 48.502943) (end 26.76 69.002943) (width 0.3) (layer "B.Cu") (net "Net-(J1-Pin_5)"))
 (segment (start 39.54 75.7) (end 40.74 74.5) (width 0.3) (layer "B.Cu") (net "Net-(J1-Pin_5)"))
 (segment (start 86.084744 78.5) (end 54.5 78.5) (width 0.3) (layer "F.Cu") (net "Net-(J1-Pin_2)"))
 (segment (start 86.7 77.884744) (end 86.084744 78.5) (width 0.3) (layer "F.Cu") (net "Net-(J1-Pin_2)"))
 (segment (start 85 71.5) (end 86.7 73.2) (width 0.3) (layer "F.Cu") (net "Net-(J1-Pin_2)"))
 (segment (start 86.7 73.2) (end 86.7 77.884744) (width 0.3) (layer "F.Cu") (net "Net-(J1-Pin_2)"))
 (via (at 54.5 78.5) (size 0.6) (drill 0.3) (layers "F.Cu" "B.Cu") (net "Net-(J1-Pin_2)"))
 (segment (start 47.28 78.5) (end 43.28 74.5) (width 0.3) (layer "B.Cu") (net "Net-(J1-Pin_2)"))
 (segment (start 54.5 78.5) (end 47.28 78.5) (width 0.3) (layer "B.Cu") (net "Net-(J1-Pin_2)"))
 (segment (start 68 75.85) (end 82.35 61.5) (width 0.3) (layer "F.Cu") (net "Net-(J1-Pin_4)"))
 (segment (start 82.35 61.5) (end 85 61.5) (width 0.3) (layer "F.Cu") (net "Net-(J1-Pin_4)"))
 (via (at 68 75.85) (size 0.6) (drill 0.3) (layers "F.Cu" "B.Cu") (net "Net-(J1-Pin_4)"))
 (segment (start 45.622943 76) (end 44.5 74.877057) (width 0.3) (layer "B.Cu") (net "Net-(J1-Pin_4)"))
 (segment (start 43.777057 73.3) (end 24.16 73.3) (width 0.3) (layer "B.Cu") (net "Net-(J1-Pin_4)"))
 (segment (start 67.85 76) (end 45.622943 76) (width 0.3) (layer "B.Cu") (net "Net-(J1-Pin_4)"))
 (segment (start 24.16 73.3) (end 22.96 74.5) (width 0.3) (layer "B.Cu") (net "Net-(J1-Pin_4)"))
 (segment (start 44.5 74.877057) (end 44.5 74.022943) (width 0.3) (layer "B.Cu") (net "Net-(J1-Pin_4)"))
 (segment (start 44.5 74.022943) (end 43.777057 73.3) (width 0.3) (layer "B.Cu") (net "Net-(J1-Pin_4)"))
 (segment (start 68 75.85) (end 67.85 76) (width 0.3) (layer "B.Cu") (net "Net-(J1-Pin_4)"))
 (segment (start 79.5 32) (end 85 26.5) (width 0.3) (layer "F.Cu") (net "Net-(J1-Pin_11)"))
 (segment (start 63.5 43.94) (end 58.44 49) (width 0.3) (layer "F.Cu") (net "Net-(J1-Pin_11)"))
 (segment (start 71 32) (end 79.5 32) (width 0.3) (layer "F.Cu") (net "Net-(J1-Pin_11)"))
 (segment (start 63.5 39.5) (end 63.5 43.94) (width 0.3) (layer "F.Cu") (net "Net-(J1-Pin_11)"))
 (via (at 71 32) (size 0.6) (drill 0.3) (layers "F.Cu" "B.Cu") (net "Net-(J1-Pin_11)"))
 (via (at 63.5 39.5) (size 0.6) (drill 0.3) (layers "F.Cu" "B.Cu") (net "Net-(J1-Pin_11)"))
 (segment (start 63.5 38.5) (end 63.5 39.5) (width 0.3) (layer "B.Cu") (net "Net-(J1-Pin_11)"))
 (segment (start 71 32) (end 70 32) (width 0.3) (layer "B.Cu") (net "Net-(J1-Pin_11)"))
 (segment (start 70 32) (end 63.5 38.5) (width 0.3) (layer "B.Cu") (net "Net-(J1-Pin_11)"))
 (segment (start 47 50.26) (end 45.74 49) (width 0.3) (layer "F.Cu") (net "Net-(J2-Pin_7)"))
 (segment (start 59.5 105.75) (end 47 93.25) (width 0.3) (layer "F.Cu") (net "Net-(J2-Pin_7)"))
 (segment (start 47 93.25) (end 47 50.26) (width 0.3) (layer "F.Cu") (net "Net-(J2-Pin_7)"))
 (segment (start 59.5 101.7) (end 52.29 94.49) (width 0.3) (layer "F.Cu") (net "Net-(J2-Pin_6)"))
 (segment (start 52.29 94.49) (end 52.29 53.01) (width 0.3) (layer "F.Cu") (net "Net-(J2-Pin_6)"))
 (segment (start 52.29 53.01) (end 48.28 49) (width 0.3) (layer "F.Cu") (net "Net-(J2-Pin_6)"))
 (segment (start 76.92 13) (end 67.92 22) (width 0.5) (layer "F.Cu") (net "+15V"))
 (segment (start 79 110.5) (end 87.5 110.5) (width 0.5) (layer "F.Cu") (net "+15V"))
 (segment (start 87.5 110.5) (end 90.5 107.5) (width 0.5) (layer "F.Cu") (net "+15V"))
 (segment (start 90.5 16.5) (end 87 13) (width 0.5) (layer "F.Cu") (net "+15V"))
 (segment (start 90.5 107.5) (end 90.5 16.5) (width 0.5) (layer "F.Cu") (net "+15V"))
 (segment (start 87 13) (end 76.92 13) (width 0.5) (layer "F.Cu") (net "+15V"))
 (segment (start 68 99.5) (end 79 110.5) (width 0.5) (layer "F.Cu") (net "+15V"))
 (segment (start 71.121321 17.5) (end 68 17.5) (width 0.5) (layer "B.Cu") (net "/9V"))
 (segment (start 68 17.5) (end 66 19.5) (width 0.5) (layer "B.Cu") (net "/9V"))
 (segment (start 66 19.5) (end 66 25.833453) (width 0.5) (layer "B.Cu") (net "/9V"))
 (segment (start 73 19.378679) (end 71.121321 17.5) (width 0.5) (layer "B.Cu") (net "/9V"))
 (segment (start 79.816547 39.65) (end 86.15 39.65) (width 0.5) (layer "B.Cu") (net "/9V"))
 (segment (start 73 22) (end 73 19.378679) (width 0.5) (layer "B.Cu") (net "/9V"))
 (segment (start 66 25.833453) (end 79.816547 39.65) (width 0.5) (layer "B.Cu") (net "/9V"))
 (segment (start 90.5 44) (end 90.5 79.5) (width 0.5) (layer "B.Cu") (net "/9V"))
 (segment (start 90.5 79.5) (end 85 85) (width 0.5) (layer "B.Cu") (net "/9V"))
 (segment (start 86.15 39.65) (end 90.5 44) (width 0.5) (layer "B.Cu") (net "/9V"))
 (segment (start 82.5 102.5) (end 85 105) (width 0.5) (layer "F.Cu") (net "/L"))
 (segment (start 58.25 86.75) (end 58.25 90.25) (width 0.5) (layer "F.Cu") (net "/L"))
 (segment (start 58.25 90.25) (end 64 96) (width 0.5) (layer "F.Cu") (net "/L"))
 (segment (start 80 96) (end 82.5 98.5) (width 0.5) (layer "F.Cu") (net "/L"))
 (segment (start 82.5 98.5) (end 82.5 102.5) (width 0.5) (layer "F.Cu") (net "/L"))
 (segment (start 64 96) (end 80 96) (width 0.5) (layer "F.Cu") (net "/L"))
 (segment (start 59.5 85.5) (end 58.25 86.75) (width 0.5) (layer "F.Cu") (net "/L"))
 (segment (start 85 95) (end 64.95 95) (width 0.5) (layer "F.Cu") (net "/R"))
 (segment (start 64.95 95) (end 59.5 89.55) (width 0.5) (layer "F.Cu") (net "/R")))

